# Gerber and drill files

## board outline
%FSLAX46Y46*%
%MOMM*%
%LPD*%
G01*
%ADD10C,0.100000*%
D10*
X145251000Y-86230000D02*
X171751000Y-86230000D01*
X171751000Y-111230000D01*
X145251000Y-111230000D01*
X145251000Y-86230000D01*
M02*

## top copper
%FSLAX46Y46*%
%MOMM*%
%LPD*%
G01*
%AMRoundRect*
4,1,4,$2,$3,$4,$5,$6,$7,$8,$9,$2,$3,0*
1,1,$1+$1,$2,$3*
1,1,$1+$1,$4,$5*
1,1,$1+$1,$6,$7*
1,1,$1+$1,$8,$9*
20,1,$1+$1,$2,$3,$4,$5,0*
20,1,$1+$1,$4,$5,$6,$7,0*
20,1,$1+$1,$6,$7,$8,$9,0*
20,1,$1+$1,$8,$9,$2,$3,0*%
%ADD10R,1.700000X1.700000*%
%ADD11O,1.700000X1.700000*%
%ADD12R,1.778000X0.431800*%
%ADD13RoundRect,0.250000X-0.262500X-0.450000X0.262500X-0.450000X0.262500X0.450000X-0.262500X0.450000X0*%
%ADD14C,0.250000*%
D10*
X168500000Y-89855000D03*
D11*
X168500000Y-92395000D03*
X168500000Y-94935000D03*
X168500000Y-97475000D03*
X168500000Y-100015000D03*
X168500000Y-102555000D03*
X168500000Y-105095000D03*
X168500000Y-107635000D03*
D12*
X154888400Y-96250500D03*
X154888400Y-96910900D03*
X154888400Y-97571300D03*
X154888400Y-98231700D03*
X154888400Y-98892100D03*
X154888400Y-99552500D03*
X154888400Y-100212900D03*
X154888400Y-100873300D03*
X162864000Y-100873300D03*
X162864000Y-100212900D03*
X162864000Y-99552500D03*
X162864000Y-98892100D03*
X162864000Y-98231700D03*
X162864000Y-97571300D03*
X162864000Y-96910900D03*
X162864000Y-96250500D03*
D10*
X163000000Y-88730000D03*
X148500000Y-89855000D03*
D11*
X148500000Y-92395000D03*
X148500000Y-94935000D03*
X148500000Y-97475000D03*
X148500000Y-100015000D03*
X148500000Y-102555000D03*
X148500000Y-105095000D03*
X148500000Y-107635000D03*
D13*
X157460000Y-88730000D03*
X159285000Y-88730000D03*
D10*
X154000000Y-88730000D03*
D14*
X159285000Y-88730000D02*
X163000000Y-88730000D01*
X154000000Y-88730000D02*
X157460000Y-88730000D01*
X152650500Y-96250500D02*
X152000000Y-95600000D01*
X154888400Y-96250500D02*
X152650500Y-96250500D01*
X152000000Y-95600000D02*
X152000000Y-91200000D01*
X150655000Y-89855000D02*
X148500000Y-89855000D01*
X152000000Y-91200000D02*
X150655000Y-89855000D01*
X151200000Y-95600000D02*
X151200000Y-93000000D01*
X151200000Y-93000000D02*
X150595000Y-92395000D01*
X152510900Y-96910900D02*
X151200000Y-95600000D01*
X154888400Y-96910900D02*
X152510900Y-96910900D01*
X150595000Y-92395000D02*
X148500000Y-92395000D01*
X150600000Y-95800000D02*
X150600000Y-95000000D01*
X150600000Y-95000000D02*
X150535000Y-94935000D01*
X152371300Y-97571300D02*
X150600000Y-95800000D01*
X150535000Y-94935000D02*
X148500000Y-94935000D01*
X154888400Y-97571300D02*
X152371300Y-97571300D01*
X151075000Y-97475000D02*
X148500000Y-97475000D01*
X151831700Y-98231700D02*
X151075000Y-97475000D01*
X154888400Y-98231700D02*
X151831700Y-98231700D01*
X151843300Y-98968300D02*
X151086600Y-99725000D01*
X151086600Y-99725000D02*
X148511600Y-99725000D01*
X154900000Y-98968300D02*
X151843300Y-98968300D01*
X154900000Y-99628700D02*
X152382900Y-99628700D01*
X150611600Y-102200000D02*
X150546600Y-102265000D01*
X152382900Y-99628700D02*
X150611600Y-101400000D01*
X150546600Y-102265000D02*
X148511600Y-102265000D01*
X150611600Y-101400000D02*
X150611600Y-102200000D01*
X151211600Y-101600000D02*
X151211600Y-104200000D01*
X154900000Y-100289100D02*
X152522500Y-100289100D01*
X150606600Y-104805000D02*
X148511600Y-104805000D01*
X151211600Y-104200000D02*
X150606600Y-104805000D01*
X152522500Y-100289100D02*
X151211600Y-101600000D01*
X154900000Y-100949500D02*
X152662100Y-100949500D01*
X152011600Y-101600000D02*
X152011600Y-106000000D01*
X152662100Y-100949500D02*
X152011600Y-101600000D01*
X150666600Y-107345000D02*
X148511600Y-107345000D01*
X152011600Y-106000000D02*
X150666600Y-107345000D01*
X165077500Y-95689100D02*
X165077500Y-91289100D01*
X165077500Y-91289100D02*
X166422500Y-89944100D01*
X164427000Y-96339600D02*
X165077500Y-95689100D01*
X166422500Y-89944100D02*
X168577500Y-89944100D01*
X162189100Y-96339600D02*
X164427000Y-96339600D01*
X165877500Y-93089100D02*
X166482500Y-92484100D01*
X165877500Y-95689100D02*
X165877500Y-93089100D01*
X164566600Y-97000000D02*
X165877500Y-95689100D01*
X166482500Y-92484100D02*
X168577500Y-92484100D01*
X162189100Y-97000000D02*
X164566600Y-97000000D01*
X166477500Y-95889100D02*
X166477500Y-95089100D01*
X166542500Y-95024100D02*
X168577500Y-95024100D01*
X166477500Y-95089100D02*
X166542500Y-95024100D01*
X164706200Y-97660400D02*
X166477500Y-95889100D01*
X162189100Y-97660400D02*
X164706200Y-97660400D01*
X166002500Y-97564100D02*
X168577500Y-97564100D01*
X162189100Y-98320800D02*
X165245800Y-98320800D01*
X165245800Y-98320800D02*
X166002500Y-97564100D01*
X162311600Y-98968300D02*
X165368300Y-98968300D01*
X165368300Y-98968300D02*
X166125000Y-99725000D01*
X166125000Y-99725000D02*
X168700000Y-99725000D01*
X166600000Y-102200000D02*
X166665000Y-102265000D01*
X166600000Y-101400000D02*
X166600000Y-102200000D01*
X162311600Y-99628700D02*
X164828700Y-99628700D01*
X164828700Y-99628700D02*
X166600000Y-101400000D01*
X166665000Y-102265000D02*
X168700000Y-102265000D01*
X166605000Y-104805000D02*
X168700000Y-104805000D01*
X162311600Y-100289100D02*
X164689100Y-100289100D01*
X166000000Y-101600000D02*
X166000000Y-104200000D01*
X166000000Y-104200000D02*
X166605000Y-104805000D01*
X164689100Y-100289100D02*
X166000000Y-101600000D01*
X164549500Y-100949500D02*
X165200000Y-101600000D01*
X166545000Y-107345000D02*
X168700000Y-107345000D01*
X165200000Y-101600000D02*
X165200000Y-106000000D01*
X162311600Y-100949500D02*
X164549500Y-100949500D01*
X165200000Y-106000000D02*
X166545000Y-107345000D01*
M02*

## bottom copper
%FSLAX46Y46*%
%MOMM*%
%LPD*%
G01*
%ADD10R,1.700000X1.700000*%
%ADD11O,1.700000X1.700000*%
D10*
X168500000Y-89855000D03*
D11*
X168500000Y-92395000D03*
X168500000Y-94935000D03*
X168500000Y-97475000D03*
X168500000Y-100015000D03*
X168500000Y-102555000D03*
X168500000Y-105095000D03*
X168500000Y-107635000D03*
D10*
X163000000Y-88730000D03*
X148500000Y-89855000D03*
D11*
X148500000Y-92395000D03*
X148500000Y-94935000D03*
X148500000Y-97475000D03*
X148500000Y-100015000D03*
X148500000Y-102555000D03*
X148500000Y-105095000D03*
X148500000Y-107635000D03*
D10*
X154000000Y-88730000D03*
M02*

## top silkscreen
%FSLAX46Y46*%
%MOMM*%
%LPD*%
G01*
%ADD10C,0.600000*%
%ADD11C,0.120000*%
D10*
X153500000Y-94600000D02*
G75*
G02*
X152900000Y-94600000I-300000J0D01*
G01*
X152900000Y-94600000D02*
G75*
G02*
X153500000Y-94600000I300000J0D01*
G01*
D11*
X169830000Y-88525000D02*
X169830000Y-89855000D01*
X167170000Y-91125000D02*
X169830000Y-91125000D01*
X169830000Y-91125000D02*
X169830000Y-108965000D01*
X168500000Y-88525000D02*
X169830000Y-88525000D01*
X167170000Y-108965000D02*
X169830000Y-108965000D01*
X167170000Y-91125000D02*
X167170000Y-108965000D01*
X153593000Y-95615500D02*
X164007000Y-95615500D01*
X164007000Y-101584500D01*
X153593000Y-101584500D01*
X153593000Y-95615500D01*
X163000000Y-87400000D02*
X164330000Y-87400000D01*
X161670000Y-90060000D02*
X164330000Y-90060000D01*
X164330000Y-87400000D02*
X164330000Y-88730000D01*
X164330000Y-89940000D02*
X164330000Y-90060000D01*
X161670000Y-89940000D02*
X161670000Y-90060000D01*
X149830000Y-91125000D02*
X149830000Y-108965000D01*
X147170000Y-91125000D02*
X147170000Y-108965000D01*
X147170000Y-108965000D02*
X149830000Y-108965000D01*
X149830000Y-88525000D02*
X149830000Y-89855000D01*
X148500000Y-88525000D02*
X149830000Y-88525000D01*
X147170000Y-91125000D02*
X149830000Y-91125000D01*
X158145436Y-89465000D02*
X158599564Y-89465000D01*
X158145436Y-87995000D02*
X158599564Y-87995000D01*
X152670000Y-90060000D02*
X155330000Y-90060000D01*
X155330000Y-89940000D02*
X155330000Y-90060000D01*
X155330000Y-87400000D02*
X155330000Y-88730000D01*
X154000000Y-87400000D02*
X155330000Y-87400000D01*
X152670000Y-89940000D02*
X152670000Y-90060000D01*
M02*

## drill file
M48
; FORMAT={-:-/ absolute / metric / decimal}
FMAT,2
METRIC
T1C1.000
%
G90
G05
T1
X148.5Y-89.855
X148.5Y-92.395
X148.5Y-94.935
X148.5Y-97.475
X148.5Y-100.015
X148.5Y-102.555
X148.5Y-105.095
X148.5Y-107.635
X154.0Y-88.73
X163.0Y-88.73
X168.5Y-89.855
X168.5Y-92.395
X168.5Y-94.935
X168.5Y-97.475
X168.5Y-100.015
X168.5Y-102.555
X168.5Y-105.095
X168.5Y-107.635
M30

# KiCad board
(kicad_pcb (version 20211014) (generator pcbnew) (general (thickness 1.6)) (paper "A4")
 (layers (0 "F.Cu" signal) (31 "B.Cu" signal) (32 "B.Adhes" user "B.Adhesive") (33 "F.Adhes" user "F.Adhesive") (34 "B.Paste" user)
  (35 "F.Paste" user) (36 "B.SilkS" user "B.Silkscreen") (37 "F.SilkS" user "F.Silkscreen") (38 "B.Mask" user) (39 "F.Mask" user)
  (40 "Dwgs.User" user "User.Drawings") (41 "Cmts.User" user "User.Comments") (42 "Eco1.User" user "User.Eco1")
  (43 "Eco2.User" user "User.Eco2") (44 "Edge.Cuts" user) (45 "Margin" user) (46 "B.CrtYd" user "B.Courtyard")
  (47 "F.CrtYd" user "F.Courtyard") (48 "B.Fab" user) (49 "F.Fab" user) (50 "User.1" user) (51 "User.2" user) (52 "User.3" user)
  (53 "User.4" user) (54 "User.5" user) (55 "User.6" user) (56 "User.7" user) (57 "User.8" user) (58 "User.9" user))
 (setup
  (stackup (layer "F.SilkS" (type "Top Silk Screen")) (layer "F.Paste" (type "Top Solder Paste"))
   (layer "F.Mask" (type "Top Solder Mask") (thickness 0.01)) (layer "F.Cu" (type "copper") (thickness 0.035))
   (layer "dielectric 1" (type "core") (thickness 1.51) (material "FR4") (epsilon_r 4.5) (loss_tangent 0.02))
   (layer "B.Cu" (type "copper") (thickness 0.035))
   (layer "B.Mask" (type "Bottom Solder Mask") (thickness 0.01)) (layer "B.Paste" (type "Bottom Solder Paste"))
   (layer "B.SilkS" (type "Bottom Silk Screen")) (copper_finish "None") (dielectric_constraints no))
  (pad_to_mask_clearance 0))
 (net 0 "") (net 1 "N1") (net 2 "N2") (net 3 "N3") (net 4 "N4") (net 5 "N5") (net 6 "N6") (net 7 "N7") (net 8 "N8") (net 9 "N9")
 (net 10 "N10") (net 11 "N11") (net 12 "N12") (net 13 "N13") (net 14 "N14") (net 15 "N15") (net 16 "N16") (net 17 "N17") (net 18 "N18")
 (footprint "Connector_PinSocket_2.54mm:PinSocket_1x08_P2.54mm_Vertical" (layer "F.Cu") (at 168.5 89.855)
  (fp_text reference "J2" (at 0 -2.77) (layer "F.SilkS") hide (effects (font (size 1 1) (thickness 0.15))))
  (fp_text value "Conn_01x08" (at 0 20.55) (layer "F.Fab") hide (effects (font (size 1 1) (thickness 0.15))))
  (fp_line (start 1.33 -1.33) (end 1.33 0) (layer "F.SilkS") (width 0.12))
  (fp_line (start -1.33 1.27) (end 1.33 1.27) (layer "F.SilkS") (width 0.12))
  (fp_line (start 1.33 1.27) (end 1.33 19.11) (layer "F.SilkS") (width 0.12))
  (fp_line (start 0 -1.33) (end 1.33 -1.33) (layer "F.SilkS") (width 0.12))
  (fp_line (start -1.33 19.11) (end 1.33 19.11) (layer "F.SilkS") (width 0.12))
  (fp_line (start -1.33 1.27) (end -1.33 19.11) (layer "F.SilkS") (width 0.12))
  (pad "1" thru_hole rect (at 0 0) (size 1.7 1.7) (drill 1) (layers *.Cu *.Mask) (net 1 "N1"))
  (pad "2" thru_hole oval (at 0 2.54) (size 1.7 1.7) (drill 1) (layers *.Cu *.Mask) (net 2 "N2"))
  (pad "3" thru_hole oval (at 0 5.08) (size 1.7 1.7) (drill 1) (layers *.Cu *.Mask) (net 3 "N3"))
  (pad "4" thru_hole oval (at 0 7.62) (size 1.7 1.7) (drill 1) (layers *.Cu *.Mask) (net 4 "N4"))
  (pad "5" thru_hole oval (at 0 10.16) (size 1.7 1.7) (drill 1) (layers *.Cu *.Mask) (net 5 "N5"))
  (pad "6" thru_hole oval (at 0 12.7) (size 1.7 1.7) (drill 1) (layers *.Cu *.Mask) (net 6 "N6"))
  (pad "7" thru_hole oval (at 0 15.24) (size 1.7 1.7) (drill 1) (layers *.Cu *.Mask) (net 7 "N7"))
  (pad "8" thru_hole oval (at 0 17.78) (size 1.7 1.7) (drill 1) (layers *.Cu *.Mask) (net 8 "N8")))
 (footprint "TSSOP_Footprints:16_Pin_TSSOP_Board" (layer "F.Cu") (at 158.8762 100.6066)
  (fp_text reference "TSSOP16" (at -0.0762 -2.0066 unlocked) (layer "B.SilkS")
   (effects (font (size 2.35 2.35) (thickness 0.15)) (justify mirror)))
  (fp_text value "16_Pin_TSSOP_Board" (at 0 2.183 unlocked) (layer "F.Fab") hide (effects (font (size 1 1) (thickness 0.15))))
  (fp_rect (start -5.2832 -4.9911) (end 5.1308 0.9779) (layer "F.SilkS") (width 0.12) (fill none))
  (pad "1" smd rect (at -3.9878 -4.3561) (size 1.778 0.4318) (layers "F.Cu" "F.Paste" "F.Mask") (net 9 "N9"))
  (pad "2" smd rect (at -3.9878 -3.6957) (size 1.778 0.4318) (layers "F.Cu" "F.Paste" "F.Mask") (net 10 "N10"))
  (pad "3" smd rect (at -3.9878 -3.0353) (size 1.778 0.4318) (layers "F.Cu" "F.Paste" "F.Mask") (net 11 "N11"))
  (pad "4" smd rect (at -3.9878 -2.3749) (size 1.778 0.4318) (layers "F.Cu" "F.Paste" "F.Mask") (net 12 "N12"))
  (pad "5" smd rect (at -3.9878 -1.7145) (size 1.778 0.4318) (layers "F.Cu" "F.Paste" "F.Mask") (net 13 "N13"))
  (pad "6" smd rect (at -3.9878 -1.0541) (size 1.778 0.4318) (layers "F.Cu" "F.Paste" "F.Mask") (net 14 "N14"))
  (pad "7" smd rect (at -3.9878 -0.3937) (size 1.778 0.4318) (layers "F.Cu" "F.Paste" "F.Mask") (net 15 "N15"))
  (pad "8" smd rect (at -3.9878 0.2667) (size 1.778 0.4318) (layers "F.Cu" "F.Paste" "F.Mask") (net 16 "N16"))
  (pad "9" smd rect (at 3.9878 0.2667) (size 1.778 0.4318) (layers "F.Cu" "F.Paste" "F.Mask") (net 8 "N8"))
  (pad "10" smd rect (at 3.9878 -0.3937) (size 1.778 0.4318) (layers "F.Cu" "F.Paste" "F.Mask") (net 7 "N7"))
  (pad "11" smd rect (at 3.9878 -1.0541) (size 1.778 0.4318) (layers "F.Cu" "F.Paste" "F.Mask") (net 6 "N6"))
  (pad "12" smd rect (at 3.9878 -1.7145) (size 1.778 0.4318) (layers "F.Cu" "F.Paste" "F.Mask") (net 5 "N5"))
  (pad "13" smd rect (at 3.9878 -2.3749) (size 1.778 0.4318) (layers "F.Cu" "F.Paste" "F.Mask") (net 4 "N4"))
  (pad "14" smd rect (at 3.9878 -3.0353) (size 1.778 0.4318) (layers "F.Cu" "F.Paste" "F.Mask") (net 3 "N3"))
  (pad "15" smd rect (at 3.9878 -3.6957) (size 1.778 0.4318) (layers "F.Cu" "F.Paste" "F.Mask") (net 2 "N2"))
  (pad "16" smd rect (at 3.9878 -4.3561) (size 1.778 0.4318) (layers "F.Cu" "F.Paste" "F.Mask") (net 1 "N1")))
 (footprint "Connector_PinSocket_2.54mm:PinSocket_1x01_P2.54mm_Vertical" (layer "F.Cu") (at 163 88.73)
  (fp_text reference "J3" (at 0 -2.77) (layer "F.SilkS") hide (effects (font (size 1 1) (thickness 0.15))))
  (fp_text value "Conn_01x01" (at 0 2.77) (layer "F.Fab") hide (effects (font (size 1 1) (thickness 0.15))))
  (fp_line (start 0 -1.33) (end 1.33 -1.33) (layer "F.SilkS") (width 0.12))
  (fp_line (start -1.33 1.33) (end 1.33 1.33) (layer "F.SilkS") (width 0.12))
  (fp_line (start 1.33 -1.33) (end 1.33 0) (layer "F.SilkS") (width 0.12))
  (fp_line (start 1.33 1.21) (end 1.33 1.33) (layer "F.SilkS") (width 0.12))
  (fp_line (start -1.33 1.21) (end -1.33 1.33) (layer "F.SilkS") (width 0.12))
  (pad "1" thru_hole rect (at 0 0) (size 1.7 1.7) (drill 1) (layers *.Cu *.Mask) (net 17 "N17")))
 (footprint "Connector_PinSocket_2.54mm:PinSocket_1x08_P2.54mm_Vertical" (layer "F.Cu") (at 148.5 89.855)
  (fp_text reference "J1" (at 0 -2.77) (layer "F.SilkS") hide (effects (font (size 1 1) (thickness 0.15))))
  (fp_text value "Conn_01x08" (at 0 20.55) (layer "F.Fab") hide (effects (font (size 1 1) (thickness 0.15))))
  (fp_line (start 1.33 1.27) (end 1.33 19.11) (layer "F.SilkS") (width 0.12))
  (fp_line (start -1.33 1.27) (end -1.33 19.11) (layer "F.SilkS") (width 0.12))
  (fp_line (start -1.33 19.11) (end 1.33 19.11) (layer "F.SilkS") (width 0.12))
  (fp_line (start 1.33 -1.33) (end 1.33 0) (layer "F.SilkS") (width 0.12))
  (fp_line (start 0 -1.33) (end 1.33 -1.33) (layer "F.SilkS") (width 0.12))
  (fp_line (start -1.33 1.27) (end 1.33 1.27) (layer "F.SilkS") (width 0.12))
  (pad "1" thru_hole rect (at 0 0) (size 1.7 1.7) (drill 1) (layers *.Cu *.Mask) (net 9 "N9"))
  (pad "2" thru_hole oval (at 0 2.54) (size 1.7 1.7) (drill 1) (layers *.Cu *.Mask) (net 10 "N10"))
  (pad "3" thru_hole oval (at 0 5.08) (size 1.7 1.7) (drill 1) (layers *.Cu *.Mask) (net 11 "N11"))
  (pad "4" thru_hole oval (at 0 7.62) (size 1.7 1.7) (drill 1) (layers *.Cu *.Mask) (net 12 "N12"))
  (pad "5" thru_hole oval (at 0 10.16) (size 1.7 1.7) (drill 1) (layers *.Cu *.Mask) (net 13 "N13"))
  (pad "6" thru_hole oval (at 0 12.7) (size 1.7 1.7) (drill 1) (layers *.Cu *.Mask) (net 14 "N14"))
  (pad "7" thru_hole oval (at 0 15.24) (size 1.7 1.7) (drill 1) (layers *.Cu *.Mask) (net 15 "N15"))
  (pad "8" thru_hole oval (at 0 17.78) (size 1.7 1.7) (drill 1) (layers *.Cu *.Mask) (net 16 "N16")))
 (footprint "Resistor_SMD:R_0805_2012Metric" (layer "F.Cu") (at 158.3725 88.73)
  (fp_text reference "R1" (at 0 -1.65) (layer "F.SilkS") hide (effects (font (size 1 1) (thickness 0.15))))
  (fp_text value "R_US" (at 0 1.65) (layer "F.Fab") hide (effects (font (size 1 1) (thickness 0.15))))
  (fp_line (start -0.227064 0.735) (end 0.227064 0.735) (layer "F.SilkS") (width 0.12))
  (fp_line (start -0.227064 -0.735) (end 0.227064 -0.735) (layer "F.SilkS") (width 0.12))
  (pad "1" smd roundrect (at -0.9125 0) (size 1.025 1.4) (layers "F.Cu" "F.Paste" "F.Mask") (roundrect_rratio 0.243902) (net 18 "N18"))
  (pad "2" smd roundrect (at 0.9125 0) (size 1.025 1.4) (layers "F.Cu" "F.Paste" "F.Mask") (roundrect_rratio 0.243902) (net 17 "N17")))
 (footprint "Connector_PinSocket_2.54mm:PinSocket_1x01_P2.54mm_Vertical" (layer "F.Cu") (at 154 88.73)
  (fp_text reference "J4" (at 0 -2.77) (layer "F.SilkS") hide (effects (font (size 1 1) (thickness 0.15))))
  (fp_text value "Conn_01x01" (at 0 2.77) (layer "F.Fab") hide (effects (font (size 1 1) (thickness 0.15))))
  (fp_line (start -1.33 1.33) (end 1.33 1.33) (layer "F.SilkS") (width 0.12))
  (fp_line (start 1.33 1.21) (end 1.33 1.33) (layer "F.SilkS") (width 0.12))
  (fp_line (start 1.33 -1.33) (end 1.33 0) (layer "F.SilkS") (width 0.12))
  (fp_line (start 0 -1.33) (end 1.33 -1.33) (layer "F.SilkS") (width 0.12))
  (fp_line (start -1.33 1.21) (end -1.33 1.33) (layer "F.SilkS") (width 0.12))
  (pad "1" thru_hole rect (at 0 0) (size 1.7 1.7) (drill 1) (layers *.Cu *.Mask) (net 18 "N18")))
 (gr_circle (center 153.2 94.6) (end 153.7 94.6) (layer "F.SilkS") (width 0.2) (fill solid))
 (gr_rect (start 145.251 86.23) (end 171.751 111.23) (layer "Edge.Cuts") (width 0.1) (fill none))
 (segment (start 159.285 88.73) (end 163 88.73) (width 0.25) (layer "F.Cu") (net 17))
 (segment (start 154 88.73) (end 157.46 88.73) (width 0.25) (layer "F.Cu") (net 18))
 (segment (start 152.6505 96.2505) (end 152 95.6) (width 0.25) (layer "F.Cu") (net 9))
 (segment (start 154.8884 96.2505) (end 152.6505 96.2505) (width 0.25) (layer "F.Cu") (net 9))
 (segment (start 152 95.6) (end 152 91.2) (width 0.25) (layer "F.Cu") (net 9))
 (segment (start 150.655 89.855) (end 148.5 89.855) (width 0.25) (layer "F.Cu") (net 9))
 (segment (start 152 91.2) (end 150.655 89.855) (width 0.25) (layer "F.Cu") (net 9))
 (segment (start 151.2 95.6) (end 151.2 93) (width 0.25) (layer "F.Cu") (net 10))
 (segment (start 151.2 93) (end 150.595 92.395) (width 0.25) (layer "F.Cu") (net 10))
 (segment (start 152.5109 96.9109) (end 151.2 95.6) (width 0.25) (layer "F.Cu") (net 10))
 (segment (start 154.8884 96.9109) (end 152.5109 96.9109) (width 0.25) (layer "F.Cu") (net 10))
 (segment (start 150.595 92.395) (end 148.5 92.395) (width 0.25) (layer "F.Cu") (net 10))
 (segment (start 150.6 95.8) (end 150.6 95) (width 0.25) (layer "F.Cu") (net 11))
 (segment (start 150.6 95) (end 150.535 94.935) (width 0.25) (layer "F.Cu") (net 11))
 (segment (start 152.3713 97.5713) (end 150.6 95.8) (width 0.25) (layer "F.Cu") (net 11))
 (segment (start 150.535 94.935) (end 148.5 94.935) (width 0.25) (layer "F.Cu") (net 11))
 (segment (start 154.8884 97.5713) (end 152.3713 97.5713) (width 0.25) (layer "F.Cu") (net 11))
 (segment (start 151.075 97.475) (end 148.5 97.475) (width 0.25) (layer "F.Cu") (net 12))
 (segment (start 151.8317 98.2317) (end 151.075 97.475) (width 0.25) (layer "F.Cu") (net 12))
 (segment (start 154.8884 98.2317) (end 151.8317 98.2317) (width 0.25) (layer "F.Cu") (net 12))
 (segment (start 151.8433 98.9683) (end 151.0866 99.725) (width 0.25) (layer "F.Cu") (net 13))
 (segment (start 151.0866 99.725) (end 148.5116 99.725) (width 0.25) (layer "F.Cu") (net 13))
 (segment (start 154.9 98.9683) (end 151.8433 98.9683) (width 0.25) (layer "F.Cu") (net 13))
 (segment (start 154.9 99.6287) (end 152.3829 99.6287) (width 0.25) (layer "F.Cu") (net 14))
 (segment (start 150.6116 102.2) (end 150.5466 102.265) (width 0.25) (layer "F.Cu") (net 14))
 (segment (start 152.3829 99.6287) (end 150.6116 101.4) (width 0.25) (layer "F.Cu") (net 14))
 (segment (start 150.5466 102.265) (end 148.5116 102.265) (width 0.25) (layer "F.Cu") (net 14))
 (segment (start 150.6116 101.4) (end 150.6116 102.2) (width 0.25) (layer "F.Cu") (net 14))
 (segment (start 151.2116 101.6) (end 151.2116 104.2) (width 0.25) (layer "F.Cu") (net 15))
 (segment (start 154.9 100.2891) (end 152.5225 100.2891) (width 0.25) (layer "F.Cu") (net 15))
 (segment (start 150.6066 104.805) (end 148.5116 104.805) (width 0.25) (layer "F.Cu") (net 15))
 (segment (start 151.2116 104.2) (end 150.6066 104.805) (width 0.25) (layer "F.Cu") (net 15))
 (segment (start 152.5225 100.2891) (end 151.2116 101.6) (width 0.25) (layer "F.Cu") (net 15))
 (segment (start 154.9 100.9495) (end 152.6621 100.9495) (width 0.25) (layer "F.Cu") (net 16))
 (segment (start 152.0116 101.6) (end 152.0116 106) (width 0.25) (layer "F.Cu") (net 16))
 (segment (start 152.6621 100.9495) (end 152.0116 101.6) (width 0.25) (layer "F.Cu") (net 16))
 (segment (start 150.6666 107.345) (end 148.5116 107.345) (width 0.25) (layer "F.Cu") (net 16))
 (segment (start 152.0116 106) (end 150.6666 107.345) (width 0.25) (layer "F.Cu") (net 16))
 (segment (start 165.0775 95.6891) (end 165.0775 91.2891) (width 0.25) (layer "F.Cu") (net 1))
 (segment (start 165.0775 91.2891) (end 166.4225 89.9441) (width 0.25) (layer "F.Cu") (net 1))
 (segment (start 164.427 96.3396) (end 165.0775 95.6891) (width 0.25) (layer "F.Cu") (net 1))
 (segment (start 166.4225 89.9441) (end 168.5775 89.9441) (width 0.25) (layer "F.Cu") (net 1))
 (segment (start 162.1891 96.3396) (end 164.427 96.3396) (width 0.25) (layer "F.Cu") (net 1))
 (segment (start 165.8775 93.0891) (end 166.4825 92.4841) (width 0.25) (layer "F.Cu") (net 2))
 (segment (start 165.8775 95.6891) (end 165.8775 93.0891) (width 0.25) (layer "F.Cu") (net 2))
 (segment (start 164.5666 97) (end 165.8775 95.6891) (width 0.25) (layer "F.Cu") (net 2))
 (segment (start 166.4825 92.4841) (end 168.5775 92.4841) (width 0.25) (layer "F.Cu") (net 2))
 (segment (start 162.1891 97) (end 164.5666 97) (width 0.25) (layer "F.Cu") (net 2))
 (segment (start 166.4775 95.8891) (end 166.4775 95.0891) (width 0.25) (layer "F.Cu") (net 3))
 (segment (start 166.5425 95.0241) (end 168.5775 95.0241) (width 0.25) (layer "F.Cu") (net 3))
 (segment (start 166.4775 95.0891) (end 166.5425 95.0241) (width 0.25) (layer "F.Cu") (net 3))
 (segment (start 164.7062 97.6604) (end 166.4775 95.8891) (width 0.25) (layer "F.Cu") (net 3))
 (segment (start 162.1891 97.6604) (end 164.7062 97.6604) (width 0.25) (layer "F.Cu") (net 3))
 (segment (start 166.0025 97.5641) (end 168.5775 97.5641) (width 0.25) (layer "F.Cu") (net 4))
 (segment (start 162.1891 98.3208) (end 165.2458 98.3208) (width 0.25) (layer "F.Cu") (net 4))
 (segment (start 165.2458 98.3208) (end 166.0025 97.5641) (width 0.25) (layer "F.Cu") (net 4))
 (segment (start 162.3116 98.9683) (end 165.3683 98.9683) (width 0.25) (layer "F.Cu") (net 5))
 (segment (start 165.3683 98.9683) (end 166.125 99.725) (width 0.25) (layer "F.Cu") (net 5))
 (segment (start 166.125 99.725) (end 168.7 99.725) (width 0.25) (layer "F.Cu") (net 5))
 (segment (start 166.6 102.2) (end 166.665 102.265) (width 0.25) (layer "F.Cu") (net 6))
 (segment (start 166.6 101.4) (end 166.6 102.2) (width 0.25) (layer "F.Cu") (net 6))
 (segment (start 162.3116 99.6287) (end 164.8287 99.6287) (width 0.25) (layer "F.Cu") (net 6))
 (segment (start 164.8287 99.6287) (end 166.6 101.4) (width 0.25) (layer "F.Cu") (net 6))
 (segment (start 166.665 102.265) (end 168.7 102.265) (width 0.25) (layer "F.Cu") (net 6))
 (segment (start 166.605 104.805) (end 168.7 104.805) (width 0.25) (layer "F.Cu") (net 7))
 (segment (start 162.3116 100.2891) (end 164.6891 100.2891) (width 0.25) (layer "F.Cu") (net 7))
 (segment (start 166 101.6) (end 166 104.2) (width 0.25) (layer "F.Cu") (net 7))
 (segment (start 166 104.2) (end 166.605 104.805) (width 0.25) (layer "F.Cu") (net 7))
 (segment (start 164.6891 100.2891) (end 166 101.6) (width 0.25) (layer "F.Cu") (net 7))
 (segment (start 164.5495 100.9495) (end 165.2 101.6) (width 0.25) (layer "F.Cu") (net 8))
 (segment (start 166.545 107.345) (end 168.7 107.345) (width 0.25) (layer "F.Cu") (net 8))
 (segment (start 165.2 101.6) (end 165.2 106) (width 0.25) (layer "F.Cu") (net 8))
 (segment (start 162.3116 100.9495) (end 164.5495 100.9495) (width 0.25) (layer "F.Cu") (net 8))
 (segment (start 165.2 106) (end 166.545 107.345) (width 0.25) (layer "F.Cu") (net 8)))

